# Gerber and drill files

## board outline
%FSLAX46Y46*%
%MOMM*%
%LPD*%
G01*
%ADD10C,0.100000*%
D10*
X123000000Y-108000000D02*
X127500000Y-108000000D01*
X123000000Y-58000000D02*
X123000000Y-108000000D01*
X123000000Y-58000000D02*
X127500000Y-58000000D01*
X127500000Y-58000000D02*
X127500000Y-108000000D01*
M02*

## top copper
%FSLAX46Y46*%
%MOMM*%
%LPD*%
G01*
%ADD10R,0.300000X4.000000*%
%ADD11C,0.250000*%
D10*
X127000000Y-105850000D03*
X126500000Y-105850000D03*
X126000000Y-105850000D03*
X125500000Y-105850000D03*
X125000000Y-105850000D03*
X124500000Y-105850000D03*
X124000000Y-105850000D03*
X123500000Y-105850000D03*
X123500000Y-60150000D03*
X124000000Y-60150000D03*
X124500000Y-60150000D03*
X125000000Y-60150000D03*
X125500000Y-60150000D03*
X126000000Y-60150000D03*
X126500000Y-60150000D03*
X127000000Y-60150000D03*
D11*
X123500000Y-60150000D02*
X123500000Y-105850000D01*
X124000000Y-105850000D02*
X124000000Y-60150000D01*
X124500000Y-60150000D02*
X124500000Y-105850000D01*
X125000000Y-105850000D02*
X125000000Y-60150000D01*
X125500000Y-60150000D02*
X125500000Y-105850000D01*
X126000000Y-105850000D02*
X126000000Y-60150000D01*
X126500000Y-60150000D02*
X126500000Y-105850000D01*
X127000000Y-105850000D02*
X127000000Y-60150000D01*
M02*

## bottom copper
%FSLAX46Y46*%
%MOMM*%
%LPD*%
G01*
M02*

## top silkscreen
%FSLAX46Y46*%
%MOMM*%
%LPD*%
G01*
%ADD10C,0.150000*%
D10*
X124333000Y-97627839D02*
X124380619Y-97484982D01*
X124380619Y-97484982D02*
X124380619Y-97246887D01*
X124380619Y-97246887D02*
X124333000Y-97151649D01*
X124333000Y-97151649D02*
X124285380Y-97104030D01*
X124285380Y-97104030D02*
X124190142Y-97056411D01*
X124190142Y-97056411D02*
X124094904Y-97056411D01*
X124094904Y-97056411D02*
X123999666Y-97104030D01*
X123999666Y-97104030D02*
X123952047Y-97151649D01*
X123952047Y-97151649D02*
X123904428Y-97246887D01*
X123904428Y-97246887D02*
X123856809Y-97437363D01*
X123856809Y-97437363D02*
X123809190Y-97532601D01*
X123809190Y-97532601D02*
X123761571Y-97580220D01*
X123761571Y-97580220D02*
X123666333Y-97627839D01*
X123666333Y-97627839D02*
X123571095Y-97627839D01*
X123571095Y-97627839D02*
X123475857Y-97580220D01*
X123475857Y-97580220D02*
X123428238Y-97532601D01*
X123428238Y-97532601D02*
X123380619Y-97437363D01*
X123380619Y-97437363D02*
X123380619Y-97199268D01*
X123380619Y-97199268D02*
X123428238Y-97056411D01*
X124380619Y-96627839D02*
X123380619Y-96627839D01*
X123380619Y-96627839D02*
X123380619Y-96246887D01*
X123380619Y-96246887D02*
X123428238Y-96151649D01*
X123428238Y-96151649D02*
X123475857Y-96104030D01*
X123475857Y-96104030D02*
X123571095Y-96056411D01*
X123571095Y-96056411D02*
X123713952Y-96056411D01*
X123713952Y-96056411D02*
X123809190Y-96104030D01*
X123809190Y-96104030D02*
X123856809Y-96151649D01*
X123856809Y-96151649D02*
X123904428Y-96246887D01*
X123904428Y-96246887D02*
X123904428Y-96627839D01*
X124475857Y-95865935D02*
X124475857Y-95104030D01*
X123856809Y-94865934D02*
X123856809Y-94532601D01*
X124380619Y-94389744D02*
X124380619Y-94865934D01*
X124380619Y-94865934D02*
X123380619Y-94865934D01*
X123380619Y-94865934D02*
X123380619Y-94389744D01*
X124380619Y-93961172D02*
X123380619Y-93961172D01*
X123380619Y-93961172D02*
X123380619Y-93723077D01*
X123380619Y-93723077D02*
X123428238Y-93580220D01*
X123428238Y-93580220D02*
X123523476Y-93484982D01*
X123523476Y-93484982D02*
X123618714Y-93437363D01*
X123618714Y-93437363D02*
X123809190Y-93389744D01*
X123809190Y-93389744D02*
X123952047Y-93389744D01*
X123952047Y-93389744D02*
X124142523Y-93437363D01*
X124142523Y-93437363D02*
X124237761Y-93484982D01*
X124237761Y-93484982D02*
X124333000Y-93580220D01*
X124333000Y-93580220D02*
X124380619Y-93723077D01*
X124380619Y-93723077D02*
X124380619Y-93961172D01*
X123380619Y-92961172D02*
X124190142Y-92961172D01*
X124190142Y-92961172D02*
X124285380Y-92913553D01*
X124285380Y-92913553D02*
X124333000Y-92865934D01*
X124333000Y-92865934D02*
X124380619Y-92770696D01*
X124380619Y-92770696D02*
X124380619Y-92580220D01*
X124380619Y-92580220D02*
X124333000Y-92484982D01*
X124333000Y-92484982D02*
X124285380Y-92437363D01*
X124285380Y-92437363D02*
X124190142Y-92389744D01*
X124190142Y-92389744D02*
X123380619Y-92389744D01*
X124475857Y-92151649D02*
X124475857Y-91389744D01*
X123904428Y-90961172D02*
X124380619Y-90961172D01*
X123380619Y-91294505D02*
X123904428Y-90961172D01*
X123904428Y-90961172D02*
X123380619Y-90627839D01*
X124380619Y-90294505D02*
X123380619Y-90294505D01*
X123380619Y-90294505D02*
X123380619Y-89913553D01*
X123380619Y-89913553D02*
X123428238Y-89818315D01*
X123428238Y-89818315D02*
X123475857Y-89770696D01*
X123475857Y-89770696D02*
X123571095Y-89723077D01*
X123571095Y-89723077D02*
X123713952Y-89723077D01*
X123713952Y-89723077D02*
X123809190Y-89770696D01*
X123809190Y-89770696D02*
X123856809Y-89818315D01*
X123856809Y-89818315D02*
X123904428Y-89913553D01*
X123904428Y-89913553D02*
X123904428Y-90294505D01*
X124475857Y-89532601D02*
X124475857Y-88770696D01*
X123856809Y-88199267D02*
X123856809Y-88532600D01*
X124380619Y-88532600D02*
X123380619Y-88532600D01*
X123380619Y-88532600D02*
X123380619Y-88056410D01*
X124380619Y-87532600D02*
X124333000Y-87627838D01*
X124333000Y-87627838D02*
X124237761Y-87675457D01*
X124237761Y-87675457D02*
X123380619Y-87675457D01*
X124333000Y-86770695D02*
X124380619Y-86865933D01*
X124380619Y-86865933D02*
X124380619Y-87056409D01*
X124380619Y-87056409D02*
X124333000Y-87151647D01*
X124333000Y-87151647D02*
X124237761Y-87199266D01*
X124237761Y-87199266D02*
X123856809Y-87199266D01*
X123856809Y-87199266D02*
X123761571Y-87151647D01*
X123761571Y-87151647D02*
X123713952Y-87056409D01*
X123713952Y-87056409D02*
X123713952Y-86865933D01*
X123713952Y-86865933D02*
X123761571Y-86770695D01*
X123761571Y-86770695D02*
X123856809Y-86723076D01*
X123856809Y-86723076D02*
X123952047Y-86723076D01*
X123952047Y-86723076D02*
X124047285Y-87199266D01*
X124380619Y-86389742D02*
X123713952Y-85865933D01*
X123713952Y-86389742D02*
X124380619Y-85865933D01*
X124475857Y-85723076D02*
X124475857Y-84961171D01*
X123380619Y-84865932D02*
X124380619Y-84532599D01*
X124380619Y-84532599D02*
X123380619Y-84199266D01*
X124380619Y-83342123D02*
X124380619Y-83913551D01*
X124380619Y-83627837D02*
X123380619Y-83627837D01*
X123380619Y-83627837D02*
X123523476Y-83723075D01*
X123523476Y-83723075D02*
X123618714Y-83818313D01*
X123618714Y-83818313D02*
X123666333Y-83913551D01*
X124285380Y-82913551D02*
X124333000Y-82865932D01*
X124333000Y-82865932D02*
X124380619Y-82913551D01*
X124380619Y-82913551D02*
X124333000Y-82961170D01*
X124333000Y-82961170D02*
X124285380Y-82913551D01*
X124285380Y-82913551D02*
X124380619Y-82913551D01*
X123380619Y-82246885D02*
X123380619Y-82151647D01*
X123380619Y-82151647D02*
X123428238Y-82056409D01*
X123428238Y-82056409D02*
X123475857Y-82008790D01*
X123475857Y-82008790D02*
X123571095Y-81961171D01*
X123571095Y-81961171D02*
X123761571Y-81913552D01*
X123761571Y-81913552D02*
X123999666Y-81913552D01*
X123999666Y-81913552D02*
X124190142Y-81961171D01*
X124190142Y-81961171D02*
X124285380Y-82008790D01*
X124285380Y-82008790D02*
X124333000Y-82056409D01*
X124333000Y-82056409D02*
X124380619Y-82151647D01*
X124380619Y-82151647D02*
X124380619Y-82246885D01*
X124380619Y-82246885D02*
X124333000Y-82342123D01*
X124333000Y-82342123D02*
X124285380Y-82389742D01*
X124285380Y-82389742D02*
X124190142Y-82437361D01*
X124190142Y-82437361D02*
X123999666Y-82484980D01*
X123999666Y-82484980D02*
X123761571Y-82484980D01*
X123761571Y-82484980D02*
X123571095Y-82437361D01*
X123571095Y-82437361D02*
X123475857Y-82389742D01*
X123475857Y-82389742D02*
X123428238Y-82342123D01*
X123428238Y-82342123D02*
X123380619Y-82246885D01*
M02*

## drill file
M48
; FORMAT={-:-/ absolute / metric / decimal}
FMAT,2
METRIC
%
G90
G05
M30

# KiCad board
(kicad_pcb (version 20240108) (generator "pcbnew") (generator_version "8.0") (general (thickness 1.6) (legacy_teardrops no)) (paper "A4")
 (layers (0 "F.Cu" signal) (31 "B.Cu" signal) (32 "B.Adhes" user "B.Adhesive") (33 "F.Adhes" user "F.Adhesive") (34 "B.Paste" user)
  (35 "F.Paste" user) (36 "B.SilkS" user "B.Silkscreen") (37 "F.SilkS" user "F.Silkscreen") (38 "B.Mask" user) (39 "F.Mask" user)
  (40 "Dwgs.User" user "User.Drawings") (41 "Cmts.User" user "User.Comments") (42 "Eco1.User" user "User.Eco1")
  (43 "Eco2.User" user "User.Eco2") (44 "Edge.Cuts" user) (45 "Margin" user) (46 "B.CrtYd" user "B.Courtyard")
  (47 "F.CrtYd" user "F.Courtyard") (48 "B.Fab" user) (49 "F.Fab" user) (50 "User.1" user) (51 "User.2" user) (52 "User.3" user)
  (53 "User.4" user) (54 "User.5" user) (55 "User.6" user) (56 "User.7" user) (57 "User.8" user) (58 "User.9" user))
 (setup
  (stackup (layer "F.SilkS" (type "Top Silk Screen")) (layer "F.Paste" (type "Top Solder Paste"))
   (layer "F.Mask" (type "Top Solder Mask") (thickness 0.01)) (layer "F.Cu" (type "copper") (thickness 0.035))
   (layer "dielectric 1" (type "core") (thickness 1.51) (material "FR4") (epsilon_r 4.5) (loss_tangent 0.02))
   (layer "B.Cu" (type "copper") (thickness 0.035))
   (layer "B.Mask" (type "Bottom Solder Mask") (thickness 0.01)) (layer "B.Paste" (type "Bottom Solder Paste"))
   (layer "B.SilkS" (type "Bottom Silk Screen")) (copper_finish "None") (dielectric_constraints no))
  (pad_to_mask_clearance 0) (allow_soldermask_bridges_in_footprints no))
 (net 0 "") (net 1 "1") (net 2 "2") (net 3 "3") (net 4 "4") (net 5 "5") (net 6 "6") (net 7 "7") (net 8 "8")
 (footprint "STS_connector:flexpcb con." (layer "F.Cu") (at 127.5 103.85 180)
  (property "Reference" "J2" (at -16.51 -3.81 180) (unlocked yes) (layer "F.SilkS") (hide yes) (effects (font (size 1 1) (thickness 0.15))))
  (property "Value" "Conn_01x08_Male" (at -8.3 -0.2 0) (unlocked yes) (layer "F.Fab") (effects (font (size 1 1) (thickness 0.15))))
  (pad "1" smd rect (at 0.5 -2 180) (size 0.3 4) (layers "F.Cu" "F.Paste" "F.Mask") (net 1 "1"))
  (pad "2" smd rect (at 1 -2 180) (size 0.3 4) (layers "F.Cu" "F.Paste" "F.Mask") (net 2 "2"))
  (pad "3" smd rect (at 1.5 -2 180) (size 0.3 4) (layers "F.Cu" "F.Paste" "F.Mask") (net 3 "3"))
  (pad "4" smd rect (at 2 -2 180) (size 0.3 4) (layers "F.Cu" "F.Paste" "F.Mask") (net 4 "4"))
  (pad "5" smd rect (at 2.5 -2 180) (size 0.3 4) (layers "F.Cu" "F.Paste" "F.Mask") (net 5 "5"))
  (pad "6" smd rect (at 3 -2 180) (size 0.3 4) (layers "F.Cu" "F.Paste" "F.Mask") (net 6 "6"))
  (pad "7" smd rect (at 3.5 -2 180) (size 0.3 4) (layers "F.Cu" "F.Paste" "F.Mask") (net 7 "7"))
  (pad "8" smd rect (at 4 -2 180) (size 0.3 4) (layers "F.Cu" "F.Paste" "F.Mask") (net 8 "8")))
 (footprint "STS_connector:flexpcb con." (layer "F.Cu") (at 123 62.15)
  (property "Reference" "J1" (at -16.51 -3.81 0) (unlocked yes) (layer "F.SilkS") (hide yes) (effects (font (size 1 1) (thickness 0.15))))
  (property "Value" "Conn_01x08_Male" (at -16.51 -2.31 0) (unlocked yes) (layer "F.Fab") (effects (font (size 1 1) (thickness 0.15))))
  (pad "1" smd rect (at 0.5 -2) (size 0.3 4) (layers "F.Cu" "F.Paste" "F.Mask") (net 8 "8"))
  (pad "2" smd rect (at 1 -2) (size 0.3 4) (layers "F.Cu" "F.Paste" "F.Mask") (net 7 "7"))
  (pad "3" smd rect (at 1.5 -2) (size 0.3 4) (layers "F.Cu" "F.Paste" "F.Mask") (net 6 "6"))
  (pad "4" smd rect (at 2 -2) (size 0.3 4) (layers "F.Cu" "F.Paste" "F.Mask") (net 5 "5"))
  (pad "5" smd rect (at 2.5 -2) (size 0.3 4) (layers "F.Cu" "F.Paste" "F.Mask") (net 4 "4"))
  (pad "6" smd rect (at 3 -2) (size 0.3 4) (layers "F.Cu" "F.Paste" "F.Mask") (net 3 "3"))
  (pad "7" smd rect (at 3.5 -2) (size 0.3 4) (layers "F.Cu" "F.Paste" "F.Mask") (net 2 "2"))
  (pad "8" smd rect (at 4 -2) (size 0.3 4) (layers "F.Cu" "F.Paste" "F.Mask") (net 1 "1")))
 (gr_line (start 123 108) (end 127.5 108) (stroke (width 0.1) (type solid)) (layer "Edge.Cuts"))
 (gr_line (start 123 58) (end 123 108) (stroke (width 0.1) (type solid)) (layer "Edge.Cuts"))
 (gr_line (start 123 58) (end 127.5 58) (stroke (width 0.1) (type solid)) (layer "Edge.Cuts"))
 (gr_line (start 127.5 58) (end 127.5 108) (stroke (width 0.1) (type solid)) (layer "Edge.Cuts"))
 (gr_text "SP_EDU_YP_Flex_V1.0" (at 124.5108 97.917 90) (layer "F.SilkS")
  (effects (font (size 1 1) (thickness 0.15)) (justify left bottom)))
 (segment (start 123.5 60.15) (end 123.5 105.85) (width 0.25) (layer "F.Cu") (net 8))
 (segment (start 124 105.85) (end 124 60.15) (width 0.25) (layer "F.Cu") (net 7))
 (segment (start 124.5 60.15) (end 124.5 105.85) (width 0.25) (layer "F.Cu") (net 6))
 (segment (start 125 105.85) (end 125 60.15) (width 0.25) (layer "F.Cu") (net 5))
 (segment (start 125.5 60.15) (end 125.5 105.85) (width 0.25) (layer "F.Cu") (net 4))
 (segment (start 126 105.85) (end 126 60.15) (width 0.25) (layer "F.Cu") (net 3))
 (segment (start 126.5 60.15) (end 126.5 105.85) (width 0.25) (layer "F.Cu") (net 2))
 (segment (start 127 105.85) (end 127 60.15) (width 0.25) (layer "F.Cu") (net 1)))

